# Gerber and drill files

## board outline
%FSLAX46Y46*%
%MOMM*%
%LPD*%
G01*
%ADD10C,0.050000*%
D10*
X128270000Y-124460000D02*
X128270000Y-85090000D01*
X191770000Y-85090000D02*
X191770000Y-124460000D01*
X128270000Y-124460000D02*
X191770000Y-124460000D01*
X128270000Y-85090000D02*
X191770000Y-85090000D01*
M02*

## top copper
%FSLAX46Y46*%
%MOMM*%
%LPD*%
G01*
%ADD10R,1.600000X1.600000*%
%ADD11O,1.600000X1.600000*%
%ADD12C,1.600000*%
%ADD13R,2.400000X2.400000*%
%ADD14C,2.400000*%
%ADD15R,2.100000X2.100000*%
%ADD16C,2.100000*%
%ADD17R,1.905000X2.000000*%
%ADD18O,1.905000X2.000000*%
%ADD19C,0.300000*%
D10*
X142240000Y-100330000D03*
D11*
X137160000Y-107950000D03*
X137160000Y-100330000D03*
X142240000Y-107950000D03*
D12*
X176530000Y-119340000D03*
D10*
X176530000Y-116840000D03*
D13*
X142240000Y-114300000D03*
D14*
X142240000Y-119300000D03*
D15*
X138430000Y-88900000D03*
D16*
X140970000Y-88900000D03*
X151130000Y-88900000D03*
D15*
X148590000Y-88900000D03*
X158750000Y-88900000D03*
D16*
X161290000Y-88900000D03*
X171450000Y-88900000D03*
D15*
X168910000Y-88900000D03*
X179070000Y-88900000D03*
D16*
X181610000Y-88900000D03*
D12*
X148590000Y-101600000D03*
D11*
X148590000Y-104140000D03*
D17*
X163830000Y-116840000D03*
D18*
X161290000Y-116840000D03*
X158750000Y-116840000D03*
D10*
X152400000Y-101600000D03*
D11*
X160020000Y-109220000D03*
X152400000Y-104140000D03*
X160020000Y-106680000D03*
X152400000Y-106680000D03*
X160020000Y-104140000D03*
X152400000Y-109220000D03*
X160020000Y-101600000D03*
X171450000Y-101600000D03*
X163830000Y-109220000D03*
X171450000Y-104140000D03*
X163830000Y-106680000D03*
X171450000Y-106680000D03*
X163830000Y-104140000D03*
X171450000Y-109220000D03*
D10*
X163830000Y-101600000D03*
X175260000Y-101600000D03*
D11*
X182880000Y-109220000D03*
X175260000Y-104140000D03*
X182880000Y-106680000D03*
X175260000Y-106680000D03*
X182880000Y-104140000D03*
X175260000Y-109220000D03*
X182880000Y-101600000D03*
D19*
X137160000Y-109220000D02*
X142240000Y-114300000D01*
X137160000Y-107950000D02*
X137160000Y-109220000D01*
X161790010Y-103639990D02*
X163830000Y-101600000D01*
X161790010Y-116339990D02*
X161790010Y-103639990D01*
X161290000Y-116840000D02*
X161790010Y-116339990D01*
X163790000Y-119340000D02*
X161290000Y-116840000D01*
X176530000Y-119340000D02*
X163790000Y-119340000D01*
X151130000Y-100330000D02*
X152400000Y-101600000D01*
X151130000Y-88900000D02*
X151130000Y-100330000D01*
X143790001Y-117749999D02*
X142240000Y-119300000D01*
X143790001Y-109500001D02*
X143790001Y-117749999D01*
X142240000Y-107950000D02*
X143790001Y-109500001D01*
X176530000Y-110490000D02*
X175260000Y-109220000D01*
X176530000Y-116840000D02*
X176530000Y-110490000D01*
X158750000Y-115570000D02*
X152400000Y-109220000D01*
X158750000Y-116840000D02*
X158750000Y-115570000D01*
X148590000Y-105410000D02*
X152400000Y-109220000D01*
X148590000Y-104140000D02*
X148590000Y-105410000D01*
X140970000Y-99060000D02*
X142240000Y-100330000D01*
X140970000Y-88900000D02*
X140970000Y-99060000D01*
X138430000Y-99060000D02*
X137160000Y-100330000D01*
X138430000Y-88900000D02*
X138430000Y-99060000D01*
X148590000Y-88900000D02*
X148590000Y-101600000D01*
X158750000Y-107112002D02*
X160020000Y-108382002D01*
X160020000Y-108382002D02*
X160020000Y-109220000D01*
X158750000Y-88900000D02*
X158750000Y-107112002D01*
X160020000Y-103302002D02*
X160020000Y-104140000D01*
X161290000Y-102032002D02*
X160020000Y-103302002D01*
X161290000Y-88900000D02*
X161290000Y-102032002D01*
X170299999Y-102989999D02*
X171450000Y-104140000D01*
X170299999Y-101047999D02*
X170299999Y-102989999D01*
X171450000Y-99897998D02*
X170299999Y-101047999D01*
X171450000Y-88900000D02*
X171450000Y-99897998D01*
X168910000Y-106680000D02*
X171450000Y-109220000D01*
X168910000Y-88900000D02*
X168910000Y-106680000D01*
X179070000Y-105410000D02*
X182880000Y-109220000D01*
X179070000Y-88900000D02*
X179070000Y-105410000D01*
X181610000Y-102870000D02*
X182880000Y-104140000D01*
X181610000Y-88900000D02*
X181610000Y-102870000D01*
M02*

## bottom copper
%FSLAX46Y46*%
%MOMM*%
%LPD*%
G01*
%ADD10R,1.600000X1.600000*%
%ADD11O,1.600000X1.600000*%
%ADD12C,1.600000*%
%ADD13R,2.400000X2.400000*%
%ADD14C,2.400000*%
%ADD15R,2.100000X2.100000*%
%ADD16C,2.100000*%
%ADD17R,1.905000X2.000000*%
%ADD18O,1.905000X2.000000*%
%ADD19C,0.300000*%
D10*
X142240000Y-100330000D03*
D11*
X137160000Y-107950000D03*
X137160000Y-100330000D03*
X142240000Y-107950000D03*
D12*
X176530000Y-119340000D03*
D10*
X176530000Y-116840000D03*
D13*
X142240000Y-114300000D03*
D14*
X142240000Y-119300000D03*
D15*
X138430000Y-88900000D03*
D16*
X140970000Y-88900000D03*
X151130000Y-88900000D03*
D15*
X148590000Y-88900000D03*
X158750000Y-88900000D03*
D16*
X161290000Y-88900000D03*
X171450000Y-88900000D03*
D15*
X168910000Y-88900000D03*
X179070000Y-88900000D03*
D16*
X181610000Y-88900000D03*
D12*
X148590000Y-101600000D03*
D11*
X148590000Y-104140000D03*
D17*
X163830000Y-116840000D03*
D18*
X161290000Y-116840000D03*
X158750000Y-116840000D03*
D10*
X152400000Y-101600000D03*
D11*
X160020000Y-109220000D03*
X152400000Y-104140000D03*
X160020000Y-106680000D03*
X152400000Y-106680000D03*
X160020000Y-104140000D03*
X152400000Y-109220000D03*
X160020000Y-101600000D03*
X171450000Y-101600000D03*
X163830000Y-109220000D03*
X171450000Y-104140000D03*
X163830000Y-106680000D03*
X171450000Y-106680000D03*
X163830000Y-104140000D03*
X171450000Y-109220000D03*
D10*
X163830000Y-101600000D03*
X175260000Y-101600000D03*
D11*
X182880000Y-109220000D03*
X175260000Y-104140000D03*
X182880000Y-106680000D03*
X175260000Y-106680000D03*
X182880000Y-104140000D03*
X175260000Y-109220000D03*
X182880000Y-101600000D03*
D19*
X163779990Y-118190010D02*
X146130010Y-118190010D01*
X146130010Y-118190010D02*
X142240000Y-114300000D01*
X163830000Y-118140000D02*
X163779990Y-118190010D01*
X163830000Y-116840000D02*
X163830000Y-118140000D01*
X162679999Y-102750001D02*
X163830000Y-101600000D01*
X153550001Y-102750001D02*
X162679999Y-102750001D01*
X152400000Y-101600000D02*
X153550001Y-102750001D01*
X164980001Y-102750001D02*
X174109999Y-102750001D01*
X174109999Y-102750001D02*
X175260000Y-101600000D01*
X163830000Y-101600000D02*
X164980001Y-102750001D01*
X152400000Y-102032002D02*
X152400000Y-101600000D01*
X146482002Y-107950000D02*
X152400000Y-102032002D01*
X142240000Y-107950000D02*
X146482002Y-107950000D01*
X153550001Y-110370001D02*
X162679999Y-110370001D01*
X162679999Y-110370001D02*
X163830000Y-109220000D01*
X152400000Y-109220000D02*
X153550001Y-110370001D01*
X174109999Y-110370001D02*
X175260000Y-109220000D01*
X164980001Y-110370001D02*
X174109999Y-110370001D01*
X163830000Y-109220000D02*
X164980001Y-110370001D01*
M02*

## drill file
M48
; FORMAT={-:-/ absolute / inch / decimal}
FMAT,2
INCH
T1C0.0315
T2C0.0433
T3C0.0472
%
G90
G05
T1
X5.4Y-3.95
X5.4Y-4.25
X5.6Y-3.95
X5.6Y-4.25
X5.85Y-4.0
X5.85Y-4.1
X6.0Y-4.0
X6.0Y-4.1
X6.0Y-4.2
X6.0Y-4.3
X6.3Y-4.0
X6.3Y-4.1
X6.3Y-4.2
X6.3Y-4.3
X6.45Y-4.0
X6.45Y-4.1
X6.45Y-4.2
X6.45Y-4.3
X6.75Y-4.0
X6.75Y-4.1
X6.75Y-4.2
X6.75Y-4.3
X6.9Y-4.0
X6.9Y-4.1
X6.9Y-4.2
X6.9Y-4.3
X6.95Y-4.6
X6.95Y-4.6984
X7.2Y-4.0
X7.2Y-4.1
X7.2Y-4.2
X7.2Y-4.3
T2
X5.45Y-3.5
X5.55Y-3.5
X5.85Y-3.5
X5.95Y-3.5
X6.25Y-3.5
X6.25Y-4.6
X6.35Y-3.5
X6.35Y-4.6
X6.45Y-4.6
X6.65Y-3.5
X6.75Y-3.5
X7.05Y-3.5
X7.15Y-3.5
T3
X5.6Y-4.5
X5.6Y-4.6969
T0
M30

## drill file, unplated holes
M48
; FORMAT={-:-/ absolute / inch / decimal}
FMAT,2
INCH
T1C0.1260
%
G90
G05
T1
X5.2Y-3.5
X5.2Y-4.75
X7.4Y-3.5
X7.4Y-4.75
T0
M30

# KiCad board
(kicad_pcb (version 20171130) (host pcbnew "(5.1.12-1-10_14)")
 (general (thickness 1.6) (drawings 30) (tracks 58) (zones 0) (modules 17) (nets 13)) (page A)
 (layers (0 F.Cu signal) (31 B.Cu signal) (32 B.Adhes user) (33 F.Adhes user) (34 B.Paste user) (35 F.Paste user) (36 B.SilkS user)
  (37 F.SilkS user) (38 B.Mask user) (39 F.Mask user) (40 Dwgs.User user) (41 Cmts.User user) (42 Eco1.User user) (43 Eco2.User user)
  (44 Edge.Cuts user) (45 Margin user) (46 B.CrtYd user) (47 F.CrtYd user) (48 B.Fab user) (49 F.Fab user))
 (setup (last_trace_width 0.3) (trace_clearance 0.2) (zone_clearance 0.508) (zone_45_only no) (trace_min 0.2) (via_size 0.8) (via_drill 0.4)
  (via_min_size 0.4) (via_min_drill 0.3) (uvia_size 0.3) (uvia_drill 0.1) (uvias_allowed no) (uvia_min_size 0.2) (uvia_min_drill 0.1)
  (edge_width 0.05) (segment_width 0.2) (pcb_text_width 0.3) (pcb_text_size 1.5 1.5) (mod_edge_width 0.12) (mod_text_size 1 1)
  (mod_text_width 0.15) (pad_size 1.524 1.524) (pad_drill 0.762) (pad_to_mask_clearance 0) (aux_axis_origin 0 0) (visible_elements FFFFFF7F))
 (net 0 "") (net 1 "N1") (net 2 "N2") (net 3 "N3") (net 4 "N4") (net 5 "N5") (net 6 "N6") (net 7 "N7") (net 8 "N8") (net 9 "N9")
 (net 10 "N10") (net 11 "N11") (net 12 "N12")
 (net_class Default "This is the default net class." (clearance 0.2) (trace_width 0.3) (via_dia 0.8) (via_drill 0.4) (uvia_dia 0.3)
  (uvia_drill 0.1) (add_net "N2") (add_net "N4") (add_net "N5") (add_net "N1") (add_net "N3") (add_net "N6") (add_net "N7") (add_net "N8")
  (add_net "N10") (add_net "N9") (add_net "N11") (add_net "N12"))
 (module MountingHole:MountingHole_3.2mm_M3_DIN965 (layer F.Cu) (at 132.08 120.65)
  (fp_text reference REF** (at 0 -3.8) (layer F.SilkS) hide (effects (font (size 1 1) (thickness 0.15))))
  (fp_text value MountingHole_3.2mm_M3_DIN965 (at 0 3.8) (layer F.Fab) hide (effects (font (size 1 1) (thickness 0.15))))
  (pad 1 np_thru_hole circle (at 0 0) (size 3.2 3.2) (drill 3.2) (layers *.Cu *.Mask)))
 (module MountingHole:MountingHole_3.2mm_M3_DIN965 (layer F.Cu) (at 187.96 120.65)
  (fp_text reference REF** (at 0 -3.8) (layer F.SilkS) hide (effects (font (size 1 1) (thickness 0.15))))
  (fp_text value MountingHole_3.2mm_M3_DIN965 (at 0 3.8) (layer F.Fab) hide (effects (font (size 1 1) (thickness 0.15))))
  (pad 1 np_thru_hole circle (at 0 0) (size 3.2 3.2) (drill 3.2) (layers *.Cu *.Mask)))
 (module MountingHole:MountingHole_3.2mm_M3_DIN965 (layer F.Cu) (at 132.08 88.9)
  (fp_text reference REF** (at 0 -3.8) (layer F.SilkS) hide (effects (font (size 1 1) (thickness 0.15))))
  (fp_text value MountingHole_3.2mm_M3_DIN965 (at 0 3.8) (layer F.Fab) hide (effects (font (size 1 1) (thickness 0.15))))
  (pad 1 np_thru_hole circle (at 0 0) (size 3.2 3.2) (drill 3.2) (layers *.Cu *.Mask)))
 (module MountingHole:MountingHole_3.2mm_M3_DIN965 (layer F.Cu) (at 187.96 88.9)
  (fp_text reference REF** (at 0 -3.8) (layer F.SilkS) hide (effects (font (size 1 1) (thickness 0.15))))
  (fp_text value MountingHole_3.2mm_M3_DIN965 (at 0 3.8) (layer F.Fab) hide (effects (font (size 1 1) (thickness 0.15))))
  (pad 1 np_thru_hole circle (at 0 0) (size 3.2 3.2) (drill 3.2) (layers *.Cu *.Mask)))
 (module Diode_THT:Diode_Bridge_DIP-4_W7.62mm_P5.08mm (layer F.Cu) (at 142.24 100.33 270)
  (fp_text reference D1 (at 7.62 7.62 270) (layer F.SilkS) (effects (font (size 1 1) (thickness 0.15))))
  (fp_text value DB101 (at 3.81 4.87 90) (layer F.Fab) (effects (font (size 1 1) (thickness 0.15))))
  (pad 1 thru_hole rect (at 0 0 270) (size 1.6 1.6) (drill 0.8) (layers *.Cu *.Mask) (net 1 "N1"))
  (pad 3 thru_hole oval (at 7.62 5.08 270) (size 1.6 1.6) (drill 0.8) (layers *.Cu *.Mask) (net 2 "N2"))
  (pad 2 thru_hole oval (at 0 5.08 270) (size 1.6 1.6) (drill 0.8) (layers *.Cu *.Mask) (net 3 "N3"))
  (pad 4 thru_hole oval (at 7.62 0 270) (size 1.6 1.6) (drill 0.8) (layers *.Cu *.Mask) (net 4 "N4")))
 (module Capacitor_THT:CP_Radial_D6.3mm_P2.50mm (layer F.Cu) (at 176.53 116.84 270)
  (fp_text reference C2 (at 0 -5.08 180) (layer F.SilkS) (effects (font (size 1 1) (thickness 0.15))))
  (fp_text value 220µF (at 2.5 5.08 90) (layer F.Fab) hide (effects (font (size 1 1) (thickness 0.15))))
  (pad 2 thru_hole circle (at 2.5 0 270) (size 1.6 1.6) (drill 0.8) (layers *.Cu *.Mask) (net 4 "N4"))
  (pad 1 thru_hole rect (at 0 0 270) (size 1.6 1.6) (drill 0.8) (layers *.Cu *.Mask) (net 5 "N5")))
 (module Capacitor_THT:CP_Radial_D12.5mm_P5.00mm (layer F.Cu) (at 142.24 114.3 270)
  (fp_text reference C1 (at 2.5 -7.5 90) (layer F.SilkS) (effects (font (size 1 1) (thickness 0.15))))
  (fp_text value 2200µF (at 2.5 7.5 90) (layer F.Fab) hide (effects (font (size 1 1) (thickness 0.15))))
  (pad 1 thru_hole rect (at 0 0 270) (size 2.4 2.4) (drill 1.2) (layers *.Cu *.Mask) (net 2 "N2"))
  (pad 2 thru_hole circle (at 5 0 270) (size 2.4 2.4) (drill 1.2) (layers *.Cu *.Mask) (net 4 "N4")))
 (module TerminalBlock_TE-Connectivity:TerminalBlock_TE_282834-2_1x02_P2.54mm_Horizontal (layer F.Cu) (at 138.43 88.9)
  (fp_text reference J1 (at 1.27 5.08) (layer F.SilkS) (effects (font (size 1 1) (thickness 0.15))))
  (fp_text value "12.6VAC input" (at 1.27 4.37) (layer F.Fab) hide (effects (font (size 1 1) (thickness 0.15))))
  (pad 1 thru_hole rect (at 0 0) (size 2.1 2.1) (drill 1.1) (layers *.Cu *.Mask) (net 3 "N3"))
  (pad 2 thru_hole circle (at 2.54 0) (size 2.1 2.1) (drill 1.1) (layers *.Cu *.Mask) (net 1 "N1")))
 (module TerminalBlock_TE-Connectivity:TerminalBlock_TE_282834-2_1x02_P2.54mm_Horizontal (layer F.Cu) (at 148.59 88.9)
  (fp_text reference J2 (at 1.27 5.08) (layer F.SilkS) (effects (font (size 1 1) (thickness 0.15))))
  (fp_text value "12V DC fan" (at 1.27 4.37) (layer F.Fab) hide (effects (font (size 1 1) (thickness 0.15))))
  (pad 2 thru_hole circle (at 2.54 0) (size 2.1 2.1) (drill 1.1) (layers *.Cu *.Mask) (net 4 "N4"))
  (pad 1 thru_hole rect (at 0 0) (size 2.1 2.1) (drill 1.1) (layers *.Cu *.Mask) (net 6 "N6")))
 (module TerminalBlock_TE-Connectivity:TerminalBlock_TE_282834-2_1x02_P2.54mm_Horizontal (layer F.Cu) (at 158.75 88.9)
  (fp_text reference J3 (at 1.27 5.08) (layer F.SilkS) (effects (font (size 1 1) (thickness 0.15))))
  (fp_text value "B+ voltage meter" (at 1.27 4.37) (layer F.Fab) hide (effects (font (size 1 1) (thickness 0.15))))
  (pad 1 thru_hole rect (at 0 0) (size 2.1 2.1) (drill 1.1) (layers *.Cu *.Mask) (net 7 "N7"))
  (pad 2 thru_hole circle (at 2.54 0) (size 2.1 2.1) (drill 1.1) (layers *.Cu *.Mask) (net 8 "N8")))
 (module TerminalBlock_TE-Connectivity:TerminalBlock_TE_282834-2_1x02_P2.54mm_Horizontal (layer F.Cu) (at 168.91 88.9)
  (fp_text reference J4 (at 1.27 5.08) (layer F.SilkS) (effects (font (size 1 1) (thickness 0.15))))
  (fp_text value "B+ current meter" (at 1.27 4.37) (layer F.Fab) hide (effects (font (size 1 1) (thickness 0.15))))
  (pad 2 thru_hole circle (at 2.54 0) (size 2.1 2.1) (drill 1.1) (layers *.Cu *.Mask) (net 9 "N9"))
  (pad 1 thru_hole rect (at 0 0) (size 2.1 2.1) (drill 1.1) (layers *.Cu *.Mask) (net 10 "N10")))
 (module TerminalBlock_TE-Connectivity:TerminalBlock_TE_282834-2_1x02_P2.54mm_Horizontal (layer F.Cu) (at 179.07 88.9)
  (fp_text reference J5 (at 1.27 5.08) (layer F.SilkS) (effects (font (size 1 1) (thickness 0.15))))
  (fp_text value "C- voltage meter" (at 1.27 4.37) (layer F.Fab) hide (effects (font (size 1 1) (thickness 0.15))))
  (pad 1 thru_hole rect (at 0 0) (size 2.1 2.1) (drill 1.1) (layers *.Cu *.Mask) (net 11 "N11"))
  (pad 2 thru_hole circle (at 2.54 0) (size 2.1 2.1) (drill 1.1) (layers *.Cu *.Mask) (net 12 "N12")))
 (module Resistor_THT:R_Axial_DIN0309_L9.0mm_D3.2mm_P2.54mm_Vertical (layer F.Cu) (at 148.59 101.6 270)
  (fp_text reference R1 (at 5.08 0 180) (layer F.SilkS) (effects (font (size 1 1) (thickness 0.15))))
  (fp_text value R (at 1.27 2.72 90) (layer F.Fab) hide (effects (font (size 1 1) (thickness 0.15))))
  (pad 1 thru_hole circle (at 0 0 270) (size 1.6 1.6) (drill 0.8) (layers *.Cu *.Mask) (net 6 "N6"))
  (pad 2 thru_hole oval (at 2.54 0 270) (size 1.6 1.6) (drill 0.8) (layers *.Cu *.Mask) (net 5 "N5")))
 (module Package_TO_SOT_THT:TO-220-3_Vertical (layer F.Cu) (at 163.83 116.84 180)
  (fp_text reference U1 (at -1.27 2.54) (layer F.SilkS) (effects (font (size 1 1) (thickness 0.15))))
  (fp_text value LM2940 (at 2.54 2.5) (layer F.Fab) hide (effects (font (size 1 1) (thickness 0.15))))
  (pad 1 thru_hole rect (at 0 0 180) (size 1.905 2) (drill 1.1) (layers *.Cu *.Mask) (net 2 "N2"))
  (pad 2 thru_hole oval (at 2.54 0 180) (size 1.905 2) (drill 1.1) (layers *.Cu *.Mask) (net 4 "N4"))
  (pad 3 thru_hole oval (at 5.08 0 180) (size 1.905 2) (drill 1.1) (layers *.Cu *.Mask) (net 5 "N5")))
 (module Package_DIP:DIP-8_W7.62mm (layer F.Cu) (at 152.4 101.6)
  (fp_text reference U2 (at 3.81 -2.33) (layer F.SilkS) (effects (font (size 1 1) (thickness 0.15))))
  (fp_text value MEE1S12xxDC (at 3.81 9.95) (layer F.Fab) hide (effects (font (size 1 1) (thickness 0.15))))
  (pad 1 thru_hole rect (at 0 0) (size 1.6 1.6) (drill 0.8) (layers *.Cu *.Mask) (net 4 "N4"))
  (pad 5 thru_hole oval (at 7.62 7.62) (size 1.6 1.6) (drill 0.8) (layers *.Cu *.Mask) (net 7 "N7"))
  (pad 2 thru_hole oval (at 0 2.54) (size 1.6 1.6) (drill 0.8) (layers *.Cu *.Mask))
  (pad 6 thru_hole oval (at 7.62 5.08) (size 1.6 1.6) (drill 0.8) (layers *.Cu *.Mask))
  (pad 3 thru_hole oval (at 0 5.08) (size 1.6 1.6) (drill 0.8) (layers *.Cu *.Mask))
  (pad 7 thru_hole oval (at 7.62 2.54) (size 1.6 1.6) (drill 0.8) (layers *.Cu *.Mask) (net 8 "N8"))
  (pad 4 thru_hole oval (at 0 7.62) (size 1.6 1.6) (drill 0.8) (layers *.Cu *.Mask) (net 5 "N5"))
  (pad 8 thru_hole oval (at 7.62 0) (size 1.6 1.6) (drill 0.8) (layers *.Cu *.Mask)))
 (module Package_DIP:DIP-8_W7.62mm (layer F.Cu) (at 163.83 101.6)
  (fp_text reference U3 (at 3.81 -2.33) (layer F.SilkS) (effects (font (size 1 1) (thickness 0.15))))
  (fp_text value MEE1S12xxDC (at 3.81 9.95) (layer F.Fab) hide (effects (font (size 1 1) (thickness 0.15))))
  (pad 8 thru_hole oval (at 7.62 0) (size 1.6 1.6) (drill 0.8) (layers *.Cu *.Mask))
  (pad 4 thru_hole oval (at 0 7.62) (size 1.6 1.6) (drill 0.8) (layers *.Cu *.Mask) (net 5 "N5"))
  (pad 7 thru_hole oval (at 7.62 2.54) (size 1.6 1.6) (drill 0.8) (layers *.Cu *.Mask) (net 9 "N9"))
  (pad 3 thru_hole oval (at 0 5.08) (size 1.6 1.6) (drill 0.8) (layers *.Cu *.Mask))
  (pad 6 thru_hole oval (at 7.62 5.08) (size 1.6 1.6) (drill 0.8) (layers *.Cu *.Mask))
  (pad 2 thru_hole oval (at 0 2.54) (size 1.6 1.6) (drill 0.8) (layers *.Cu *.Mask))
  (pad 5 thru_hole oval (at 7.62 7.62) (size 1.6 1.6) (drill 0.8) (layers *.Cu *.Mask) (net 10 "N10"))
  (pad 1 thru_hole rect (at 0 0) (size 1.6 1.6) (drill 0.8) (layers *.Cu *.Mask) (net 4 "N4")))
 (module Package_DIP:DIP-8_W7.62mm (layer F.Cu) (at 175.26 101.6)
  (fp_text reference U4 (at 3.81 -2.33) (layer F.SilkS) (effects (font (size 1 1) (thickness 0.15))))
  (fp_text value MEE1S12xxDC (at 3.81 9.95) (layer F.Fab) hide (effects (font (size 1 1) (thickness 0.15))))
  (pad 1 thru_hole rect (at 0 0) (size 1.6 1.6) (drill 0.8) (layers *.Cu *.Mask) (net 4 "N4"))
  (pad 5 thru_hole oval (at 7.62 7.62) (size 1.6 1.6) (drill 0.8) (layers *.Cu *.Mask) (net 11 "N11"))
  (pad 2 thru_hole oval (at 0 2.54) (size 1.6 1.6) (drill 0.8) (layers *.Cu *.Mask))
  (pad 6 thru_hole oval (at 7.62 5.08) (size 1.6 1.6) (drill 0.8) (layers *.Cu *.Mask))
  (pad 3 thru_hole oval (at 0 5.08) (size 1.6 1.6) (drill 0.8) (layers *.Cu *.Mask))
  (pad 7 thru_hole oval (at 7.62 2.54) (size 1.6 1.6) (drill 0.8) (layers *.Cu *.Mask) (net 12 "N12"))
  (pad 4 thru_hole oval (at 0 7.62) (size 1.6 1.6) (drill 0.8) (layers *.Cu *.Mask) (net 5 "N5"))
  (pad 8 thru_hole oval (at 7.62 0) (size 1.6 1.6) (drill 0.8) (layers *.Cu *.Mask)))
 (gr_line (start 128.27 124.46) (end 128.27 85.09) (layer Edge.Cuts) (width 0.05))
 (gr_line (start 191.77 85.09) (end 191.77 124.46) (layer Edge.Cuts) (width 0.05))
 (gr_line (start 128.27 124.46) (end 191.77 124.46) (layer Edge.Cuts) (width 0.05))
 (gr_line (start 128.27 85.09) (end 191.77 85.09) (layer Edge.Cuts) (width 0.05))
 (segment (start 163.77999 118.19001) (end 146.13001 118.19001) (width 0.3) (layer B.Cu) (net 2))
 (segment (start 146.13001 118.19001) (end 142.24 114.3) (width 0.3) (layer B.Cu) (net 2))
 (segment (start 163.83 118.14) (end 163.77999 118.19001) (width 0.3) (layer B.Cu) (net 2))
 (segment (start 163.83 116.84) (end 163.83 118.14) (width 0.3) (layer B.Cu) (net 2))
 (segment (start 137.16 109.22) (end 142.24 114.3) (width 0.3) (layer F.Cu) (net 2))
 (segment (start 137.16 107.95) (end 137.16 109.22) (width 0.3) (layer F.Cu) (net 2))
 (segment (start 162.679999 102.750001) (end 163.83 101.6) (width 0.3) (layer B.Cu) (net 4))
 (segment (start 153.550001 102.750001) (end 162.679999 102.750001) (width 0.3) (layer B.Cu) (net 4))
 (segment (start 152.4 101.6) (end 153.550001 102.750001) (width 0.3) (layer B.Cu) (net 4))
 (segment (start 164.980001 102.750001) (end 174.109999 102.750001) (width 0.3) (layer B.Cu) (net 4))
 (segment (start 174.109999 102.750001) (end 175.26 101.6) (width 0.3) (layer B.Cu) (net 4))
 (segment (start 163.83 101.6) (end 164.980001 102.750001) (width 0.3) (layer B.Cu) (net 4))
 (segment (start 161.79001 103.63999) (end 163.83 101.6) (width 0.3) (layer F.Cu) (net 4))
 (segment (start 161.79001 116.33999) (end 161.79001 103.63999) (width 0.3) (layer F.Cu) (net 4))
 (segment (start 161.29 116.84) (end 161.79001 116.33999) (width 0.3) (layer F.Cu) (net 4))
 (segment (start 163.79 119.34) (end 161.29 116.84) (width 0.3) (layer F.Cu) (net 4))
 (segment (start 176.53 119.34) (end 163.79 119.34) (width 0.3) (layer F.Cu) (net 4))
 (segment (start 151.13 100.33) (end 152.4 101.6) (width 0.3) (layer F.Cu) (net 4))
 (segment (start 151.13 88.9) (end 151.13 100.33) (width 0.3) (layer F.Cu) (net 4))
 (segment (start 143.790001 117.749999) (end 142.24 119.3) (width 0.3) (layer F.Cu) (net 4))
 (segment (start 143.790001 109.500001) (end 143.790001 117.749999) (width 0.3) (layer F.Cu) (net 4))
 (segment (start 142.24 107.95) (end 143.790001 109.500001) (width 0.3) (layer F.Cu) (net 4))
 (segment (start 152.4 102.032002) (end 152.4 101.6) (width 0.3) (layer B.Cu) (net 4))
 (segment (start 146.482002 107.95) (end 152.4 102.032002) (width 0.3) (layer B.Cu) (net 4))
 (segment (start 142.24 107.95) (end 146.482002 107.95) (width 0.3) (layer B.Cu) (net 4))
 (segment (start 153.550001 110.370001) (end 162.679999 110.370001) (width 0.3) (layer B.Cu) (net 5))
 (segment (start 162.679999 110.370001) (end 163.83 109.22) (width 0.3) (layer B.Cu) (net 5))
 (segment (start 152.4 109.22) (end 153.550001 110.370001) (width 0.3) (layer B.Cu) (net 5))
 (segment (start 174.109999 110.370001) (end 175.26 109.22) (width 0.3) (layer B.Cu) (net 5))
 (segment (start 164.980001 110.370001) (end 174.109999 110.370001) (width 0.3) (layer B.Cu) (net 5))
 (segment (start 163.83 109.22) (end 164.980001 110.370001) (width 0.3) (layer B.Cu) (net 5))
 (segment (start 176.53 110.49) (end 175.26 109.22) (width 0.3) (layer F.Cu) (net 5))
 (segment (start 176.53 116.84) (end 176.53 110.49) (width 0.3) (layer F.Cu) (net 5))
 (segment (start 158.75 115.57) (end 152.4 109.22) (width 0.3) (layer F.Cu) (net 5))
 (segment (start 158.75 116.84) (end 158.75 115.57) (width 0.3) (layer F.Cu) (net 5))
 (segment (start 148.59 105.41) (end 152.4 109.22) (width 0.3) (layer F.Cu) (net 5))
 (segment (start 148.59 104.14) (end 148.59 105.41) (width 0.3) (layer F.Cu) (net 5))
 (segment (start 140.97 99.06) (end 142.24 100.33) (width 0.3) (layer F.Cu) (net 1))
 (segment (start 140.97 88.9) (end 140.97 99.06) (width 0.3) (layer F.Cu) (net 1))
 (segment (start 138.43 99.06) (end 137.16 100.33) (width 0.3) (layer F.Cu) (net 3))
 (segment (start 138.43 88.9) (end 138.43 99.06) (width 0.3) (layer F.Cu) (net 3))
 (segment (start 148.59 88.9) (end 148.59 101.6) (width 0.3) (layer F.Cu) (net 6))
 (segment (start 158.75 107.112002) (end 160.02 108.382002) (width 0.3) (layer F.Cu) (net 7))
 (segment (start 160.02 108.382002) (end 160.02 109.22) (width 0.3) (layer F.Cu) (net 7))
 (segment (start 158.75 88.9) (end 158.75 107.112002) (width 0.3) (layer F.Cu) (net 7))
 (segment (start 160.02 103.302002) (end 160.02 104.14) (width 0.3) (layer F.Cu) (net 8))
 (segment (start 161.29 102.032002) (end 160.02 103.302002) (width 0.3) (layer F.Cu) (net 8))
 (segment (start 161.29 88.9) (end 161.29 102.032002) (width 0.3) (layer F.Cu) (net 8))
 (segment (start 170.299999 102.989999) (end 171.45 104.14) (width 0.3) (layer F.Cu) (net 9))
 (segment (start 170.299999 101.047999) (end 170.299999 102.989999) (width 0.3) (layer F.Cu) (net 9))
 (segment (start 171.45 99.897998) (end 170.299999 101.047999) (width 0.3) (layer F.Cu) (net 9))
 (segment (start 171.45 88.9) (end 171.45 99.897998) (width 0.3) (layer F.Cu) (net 9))
 (segment (start 168.91 106.68) (end 171.45 109.22) (width 0.3) (layer F.Cu) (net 10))
 (segment (start 168.91 88.9) (end 168.91 106.68) (width 0.3) (layer F.Cu) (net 10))
 (segment (start 179.07 105.41) (end 182.88 109.22) (width 0.3) (layer F.Cu) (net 11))
 (segment (start 179.07 88.9) (end 179.07 105.41) (width 0.3) (layer F.Cu) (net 11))
 (segment (start 181.61 102.87) (end 182.88 104.14) (width 0.3) (layer F.Cu) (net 12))
 (segment (start 181.61 88.9) (end 181.61 102.87) (width 0.3) (layer F.Cu) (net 12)))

